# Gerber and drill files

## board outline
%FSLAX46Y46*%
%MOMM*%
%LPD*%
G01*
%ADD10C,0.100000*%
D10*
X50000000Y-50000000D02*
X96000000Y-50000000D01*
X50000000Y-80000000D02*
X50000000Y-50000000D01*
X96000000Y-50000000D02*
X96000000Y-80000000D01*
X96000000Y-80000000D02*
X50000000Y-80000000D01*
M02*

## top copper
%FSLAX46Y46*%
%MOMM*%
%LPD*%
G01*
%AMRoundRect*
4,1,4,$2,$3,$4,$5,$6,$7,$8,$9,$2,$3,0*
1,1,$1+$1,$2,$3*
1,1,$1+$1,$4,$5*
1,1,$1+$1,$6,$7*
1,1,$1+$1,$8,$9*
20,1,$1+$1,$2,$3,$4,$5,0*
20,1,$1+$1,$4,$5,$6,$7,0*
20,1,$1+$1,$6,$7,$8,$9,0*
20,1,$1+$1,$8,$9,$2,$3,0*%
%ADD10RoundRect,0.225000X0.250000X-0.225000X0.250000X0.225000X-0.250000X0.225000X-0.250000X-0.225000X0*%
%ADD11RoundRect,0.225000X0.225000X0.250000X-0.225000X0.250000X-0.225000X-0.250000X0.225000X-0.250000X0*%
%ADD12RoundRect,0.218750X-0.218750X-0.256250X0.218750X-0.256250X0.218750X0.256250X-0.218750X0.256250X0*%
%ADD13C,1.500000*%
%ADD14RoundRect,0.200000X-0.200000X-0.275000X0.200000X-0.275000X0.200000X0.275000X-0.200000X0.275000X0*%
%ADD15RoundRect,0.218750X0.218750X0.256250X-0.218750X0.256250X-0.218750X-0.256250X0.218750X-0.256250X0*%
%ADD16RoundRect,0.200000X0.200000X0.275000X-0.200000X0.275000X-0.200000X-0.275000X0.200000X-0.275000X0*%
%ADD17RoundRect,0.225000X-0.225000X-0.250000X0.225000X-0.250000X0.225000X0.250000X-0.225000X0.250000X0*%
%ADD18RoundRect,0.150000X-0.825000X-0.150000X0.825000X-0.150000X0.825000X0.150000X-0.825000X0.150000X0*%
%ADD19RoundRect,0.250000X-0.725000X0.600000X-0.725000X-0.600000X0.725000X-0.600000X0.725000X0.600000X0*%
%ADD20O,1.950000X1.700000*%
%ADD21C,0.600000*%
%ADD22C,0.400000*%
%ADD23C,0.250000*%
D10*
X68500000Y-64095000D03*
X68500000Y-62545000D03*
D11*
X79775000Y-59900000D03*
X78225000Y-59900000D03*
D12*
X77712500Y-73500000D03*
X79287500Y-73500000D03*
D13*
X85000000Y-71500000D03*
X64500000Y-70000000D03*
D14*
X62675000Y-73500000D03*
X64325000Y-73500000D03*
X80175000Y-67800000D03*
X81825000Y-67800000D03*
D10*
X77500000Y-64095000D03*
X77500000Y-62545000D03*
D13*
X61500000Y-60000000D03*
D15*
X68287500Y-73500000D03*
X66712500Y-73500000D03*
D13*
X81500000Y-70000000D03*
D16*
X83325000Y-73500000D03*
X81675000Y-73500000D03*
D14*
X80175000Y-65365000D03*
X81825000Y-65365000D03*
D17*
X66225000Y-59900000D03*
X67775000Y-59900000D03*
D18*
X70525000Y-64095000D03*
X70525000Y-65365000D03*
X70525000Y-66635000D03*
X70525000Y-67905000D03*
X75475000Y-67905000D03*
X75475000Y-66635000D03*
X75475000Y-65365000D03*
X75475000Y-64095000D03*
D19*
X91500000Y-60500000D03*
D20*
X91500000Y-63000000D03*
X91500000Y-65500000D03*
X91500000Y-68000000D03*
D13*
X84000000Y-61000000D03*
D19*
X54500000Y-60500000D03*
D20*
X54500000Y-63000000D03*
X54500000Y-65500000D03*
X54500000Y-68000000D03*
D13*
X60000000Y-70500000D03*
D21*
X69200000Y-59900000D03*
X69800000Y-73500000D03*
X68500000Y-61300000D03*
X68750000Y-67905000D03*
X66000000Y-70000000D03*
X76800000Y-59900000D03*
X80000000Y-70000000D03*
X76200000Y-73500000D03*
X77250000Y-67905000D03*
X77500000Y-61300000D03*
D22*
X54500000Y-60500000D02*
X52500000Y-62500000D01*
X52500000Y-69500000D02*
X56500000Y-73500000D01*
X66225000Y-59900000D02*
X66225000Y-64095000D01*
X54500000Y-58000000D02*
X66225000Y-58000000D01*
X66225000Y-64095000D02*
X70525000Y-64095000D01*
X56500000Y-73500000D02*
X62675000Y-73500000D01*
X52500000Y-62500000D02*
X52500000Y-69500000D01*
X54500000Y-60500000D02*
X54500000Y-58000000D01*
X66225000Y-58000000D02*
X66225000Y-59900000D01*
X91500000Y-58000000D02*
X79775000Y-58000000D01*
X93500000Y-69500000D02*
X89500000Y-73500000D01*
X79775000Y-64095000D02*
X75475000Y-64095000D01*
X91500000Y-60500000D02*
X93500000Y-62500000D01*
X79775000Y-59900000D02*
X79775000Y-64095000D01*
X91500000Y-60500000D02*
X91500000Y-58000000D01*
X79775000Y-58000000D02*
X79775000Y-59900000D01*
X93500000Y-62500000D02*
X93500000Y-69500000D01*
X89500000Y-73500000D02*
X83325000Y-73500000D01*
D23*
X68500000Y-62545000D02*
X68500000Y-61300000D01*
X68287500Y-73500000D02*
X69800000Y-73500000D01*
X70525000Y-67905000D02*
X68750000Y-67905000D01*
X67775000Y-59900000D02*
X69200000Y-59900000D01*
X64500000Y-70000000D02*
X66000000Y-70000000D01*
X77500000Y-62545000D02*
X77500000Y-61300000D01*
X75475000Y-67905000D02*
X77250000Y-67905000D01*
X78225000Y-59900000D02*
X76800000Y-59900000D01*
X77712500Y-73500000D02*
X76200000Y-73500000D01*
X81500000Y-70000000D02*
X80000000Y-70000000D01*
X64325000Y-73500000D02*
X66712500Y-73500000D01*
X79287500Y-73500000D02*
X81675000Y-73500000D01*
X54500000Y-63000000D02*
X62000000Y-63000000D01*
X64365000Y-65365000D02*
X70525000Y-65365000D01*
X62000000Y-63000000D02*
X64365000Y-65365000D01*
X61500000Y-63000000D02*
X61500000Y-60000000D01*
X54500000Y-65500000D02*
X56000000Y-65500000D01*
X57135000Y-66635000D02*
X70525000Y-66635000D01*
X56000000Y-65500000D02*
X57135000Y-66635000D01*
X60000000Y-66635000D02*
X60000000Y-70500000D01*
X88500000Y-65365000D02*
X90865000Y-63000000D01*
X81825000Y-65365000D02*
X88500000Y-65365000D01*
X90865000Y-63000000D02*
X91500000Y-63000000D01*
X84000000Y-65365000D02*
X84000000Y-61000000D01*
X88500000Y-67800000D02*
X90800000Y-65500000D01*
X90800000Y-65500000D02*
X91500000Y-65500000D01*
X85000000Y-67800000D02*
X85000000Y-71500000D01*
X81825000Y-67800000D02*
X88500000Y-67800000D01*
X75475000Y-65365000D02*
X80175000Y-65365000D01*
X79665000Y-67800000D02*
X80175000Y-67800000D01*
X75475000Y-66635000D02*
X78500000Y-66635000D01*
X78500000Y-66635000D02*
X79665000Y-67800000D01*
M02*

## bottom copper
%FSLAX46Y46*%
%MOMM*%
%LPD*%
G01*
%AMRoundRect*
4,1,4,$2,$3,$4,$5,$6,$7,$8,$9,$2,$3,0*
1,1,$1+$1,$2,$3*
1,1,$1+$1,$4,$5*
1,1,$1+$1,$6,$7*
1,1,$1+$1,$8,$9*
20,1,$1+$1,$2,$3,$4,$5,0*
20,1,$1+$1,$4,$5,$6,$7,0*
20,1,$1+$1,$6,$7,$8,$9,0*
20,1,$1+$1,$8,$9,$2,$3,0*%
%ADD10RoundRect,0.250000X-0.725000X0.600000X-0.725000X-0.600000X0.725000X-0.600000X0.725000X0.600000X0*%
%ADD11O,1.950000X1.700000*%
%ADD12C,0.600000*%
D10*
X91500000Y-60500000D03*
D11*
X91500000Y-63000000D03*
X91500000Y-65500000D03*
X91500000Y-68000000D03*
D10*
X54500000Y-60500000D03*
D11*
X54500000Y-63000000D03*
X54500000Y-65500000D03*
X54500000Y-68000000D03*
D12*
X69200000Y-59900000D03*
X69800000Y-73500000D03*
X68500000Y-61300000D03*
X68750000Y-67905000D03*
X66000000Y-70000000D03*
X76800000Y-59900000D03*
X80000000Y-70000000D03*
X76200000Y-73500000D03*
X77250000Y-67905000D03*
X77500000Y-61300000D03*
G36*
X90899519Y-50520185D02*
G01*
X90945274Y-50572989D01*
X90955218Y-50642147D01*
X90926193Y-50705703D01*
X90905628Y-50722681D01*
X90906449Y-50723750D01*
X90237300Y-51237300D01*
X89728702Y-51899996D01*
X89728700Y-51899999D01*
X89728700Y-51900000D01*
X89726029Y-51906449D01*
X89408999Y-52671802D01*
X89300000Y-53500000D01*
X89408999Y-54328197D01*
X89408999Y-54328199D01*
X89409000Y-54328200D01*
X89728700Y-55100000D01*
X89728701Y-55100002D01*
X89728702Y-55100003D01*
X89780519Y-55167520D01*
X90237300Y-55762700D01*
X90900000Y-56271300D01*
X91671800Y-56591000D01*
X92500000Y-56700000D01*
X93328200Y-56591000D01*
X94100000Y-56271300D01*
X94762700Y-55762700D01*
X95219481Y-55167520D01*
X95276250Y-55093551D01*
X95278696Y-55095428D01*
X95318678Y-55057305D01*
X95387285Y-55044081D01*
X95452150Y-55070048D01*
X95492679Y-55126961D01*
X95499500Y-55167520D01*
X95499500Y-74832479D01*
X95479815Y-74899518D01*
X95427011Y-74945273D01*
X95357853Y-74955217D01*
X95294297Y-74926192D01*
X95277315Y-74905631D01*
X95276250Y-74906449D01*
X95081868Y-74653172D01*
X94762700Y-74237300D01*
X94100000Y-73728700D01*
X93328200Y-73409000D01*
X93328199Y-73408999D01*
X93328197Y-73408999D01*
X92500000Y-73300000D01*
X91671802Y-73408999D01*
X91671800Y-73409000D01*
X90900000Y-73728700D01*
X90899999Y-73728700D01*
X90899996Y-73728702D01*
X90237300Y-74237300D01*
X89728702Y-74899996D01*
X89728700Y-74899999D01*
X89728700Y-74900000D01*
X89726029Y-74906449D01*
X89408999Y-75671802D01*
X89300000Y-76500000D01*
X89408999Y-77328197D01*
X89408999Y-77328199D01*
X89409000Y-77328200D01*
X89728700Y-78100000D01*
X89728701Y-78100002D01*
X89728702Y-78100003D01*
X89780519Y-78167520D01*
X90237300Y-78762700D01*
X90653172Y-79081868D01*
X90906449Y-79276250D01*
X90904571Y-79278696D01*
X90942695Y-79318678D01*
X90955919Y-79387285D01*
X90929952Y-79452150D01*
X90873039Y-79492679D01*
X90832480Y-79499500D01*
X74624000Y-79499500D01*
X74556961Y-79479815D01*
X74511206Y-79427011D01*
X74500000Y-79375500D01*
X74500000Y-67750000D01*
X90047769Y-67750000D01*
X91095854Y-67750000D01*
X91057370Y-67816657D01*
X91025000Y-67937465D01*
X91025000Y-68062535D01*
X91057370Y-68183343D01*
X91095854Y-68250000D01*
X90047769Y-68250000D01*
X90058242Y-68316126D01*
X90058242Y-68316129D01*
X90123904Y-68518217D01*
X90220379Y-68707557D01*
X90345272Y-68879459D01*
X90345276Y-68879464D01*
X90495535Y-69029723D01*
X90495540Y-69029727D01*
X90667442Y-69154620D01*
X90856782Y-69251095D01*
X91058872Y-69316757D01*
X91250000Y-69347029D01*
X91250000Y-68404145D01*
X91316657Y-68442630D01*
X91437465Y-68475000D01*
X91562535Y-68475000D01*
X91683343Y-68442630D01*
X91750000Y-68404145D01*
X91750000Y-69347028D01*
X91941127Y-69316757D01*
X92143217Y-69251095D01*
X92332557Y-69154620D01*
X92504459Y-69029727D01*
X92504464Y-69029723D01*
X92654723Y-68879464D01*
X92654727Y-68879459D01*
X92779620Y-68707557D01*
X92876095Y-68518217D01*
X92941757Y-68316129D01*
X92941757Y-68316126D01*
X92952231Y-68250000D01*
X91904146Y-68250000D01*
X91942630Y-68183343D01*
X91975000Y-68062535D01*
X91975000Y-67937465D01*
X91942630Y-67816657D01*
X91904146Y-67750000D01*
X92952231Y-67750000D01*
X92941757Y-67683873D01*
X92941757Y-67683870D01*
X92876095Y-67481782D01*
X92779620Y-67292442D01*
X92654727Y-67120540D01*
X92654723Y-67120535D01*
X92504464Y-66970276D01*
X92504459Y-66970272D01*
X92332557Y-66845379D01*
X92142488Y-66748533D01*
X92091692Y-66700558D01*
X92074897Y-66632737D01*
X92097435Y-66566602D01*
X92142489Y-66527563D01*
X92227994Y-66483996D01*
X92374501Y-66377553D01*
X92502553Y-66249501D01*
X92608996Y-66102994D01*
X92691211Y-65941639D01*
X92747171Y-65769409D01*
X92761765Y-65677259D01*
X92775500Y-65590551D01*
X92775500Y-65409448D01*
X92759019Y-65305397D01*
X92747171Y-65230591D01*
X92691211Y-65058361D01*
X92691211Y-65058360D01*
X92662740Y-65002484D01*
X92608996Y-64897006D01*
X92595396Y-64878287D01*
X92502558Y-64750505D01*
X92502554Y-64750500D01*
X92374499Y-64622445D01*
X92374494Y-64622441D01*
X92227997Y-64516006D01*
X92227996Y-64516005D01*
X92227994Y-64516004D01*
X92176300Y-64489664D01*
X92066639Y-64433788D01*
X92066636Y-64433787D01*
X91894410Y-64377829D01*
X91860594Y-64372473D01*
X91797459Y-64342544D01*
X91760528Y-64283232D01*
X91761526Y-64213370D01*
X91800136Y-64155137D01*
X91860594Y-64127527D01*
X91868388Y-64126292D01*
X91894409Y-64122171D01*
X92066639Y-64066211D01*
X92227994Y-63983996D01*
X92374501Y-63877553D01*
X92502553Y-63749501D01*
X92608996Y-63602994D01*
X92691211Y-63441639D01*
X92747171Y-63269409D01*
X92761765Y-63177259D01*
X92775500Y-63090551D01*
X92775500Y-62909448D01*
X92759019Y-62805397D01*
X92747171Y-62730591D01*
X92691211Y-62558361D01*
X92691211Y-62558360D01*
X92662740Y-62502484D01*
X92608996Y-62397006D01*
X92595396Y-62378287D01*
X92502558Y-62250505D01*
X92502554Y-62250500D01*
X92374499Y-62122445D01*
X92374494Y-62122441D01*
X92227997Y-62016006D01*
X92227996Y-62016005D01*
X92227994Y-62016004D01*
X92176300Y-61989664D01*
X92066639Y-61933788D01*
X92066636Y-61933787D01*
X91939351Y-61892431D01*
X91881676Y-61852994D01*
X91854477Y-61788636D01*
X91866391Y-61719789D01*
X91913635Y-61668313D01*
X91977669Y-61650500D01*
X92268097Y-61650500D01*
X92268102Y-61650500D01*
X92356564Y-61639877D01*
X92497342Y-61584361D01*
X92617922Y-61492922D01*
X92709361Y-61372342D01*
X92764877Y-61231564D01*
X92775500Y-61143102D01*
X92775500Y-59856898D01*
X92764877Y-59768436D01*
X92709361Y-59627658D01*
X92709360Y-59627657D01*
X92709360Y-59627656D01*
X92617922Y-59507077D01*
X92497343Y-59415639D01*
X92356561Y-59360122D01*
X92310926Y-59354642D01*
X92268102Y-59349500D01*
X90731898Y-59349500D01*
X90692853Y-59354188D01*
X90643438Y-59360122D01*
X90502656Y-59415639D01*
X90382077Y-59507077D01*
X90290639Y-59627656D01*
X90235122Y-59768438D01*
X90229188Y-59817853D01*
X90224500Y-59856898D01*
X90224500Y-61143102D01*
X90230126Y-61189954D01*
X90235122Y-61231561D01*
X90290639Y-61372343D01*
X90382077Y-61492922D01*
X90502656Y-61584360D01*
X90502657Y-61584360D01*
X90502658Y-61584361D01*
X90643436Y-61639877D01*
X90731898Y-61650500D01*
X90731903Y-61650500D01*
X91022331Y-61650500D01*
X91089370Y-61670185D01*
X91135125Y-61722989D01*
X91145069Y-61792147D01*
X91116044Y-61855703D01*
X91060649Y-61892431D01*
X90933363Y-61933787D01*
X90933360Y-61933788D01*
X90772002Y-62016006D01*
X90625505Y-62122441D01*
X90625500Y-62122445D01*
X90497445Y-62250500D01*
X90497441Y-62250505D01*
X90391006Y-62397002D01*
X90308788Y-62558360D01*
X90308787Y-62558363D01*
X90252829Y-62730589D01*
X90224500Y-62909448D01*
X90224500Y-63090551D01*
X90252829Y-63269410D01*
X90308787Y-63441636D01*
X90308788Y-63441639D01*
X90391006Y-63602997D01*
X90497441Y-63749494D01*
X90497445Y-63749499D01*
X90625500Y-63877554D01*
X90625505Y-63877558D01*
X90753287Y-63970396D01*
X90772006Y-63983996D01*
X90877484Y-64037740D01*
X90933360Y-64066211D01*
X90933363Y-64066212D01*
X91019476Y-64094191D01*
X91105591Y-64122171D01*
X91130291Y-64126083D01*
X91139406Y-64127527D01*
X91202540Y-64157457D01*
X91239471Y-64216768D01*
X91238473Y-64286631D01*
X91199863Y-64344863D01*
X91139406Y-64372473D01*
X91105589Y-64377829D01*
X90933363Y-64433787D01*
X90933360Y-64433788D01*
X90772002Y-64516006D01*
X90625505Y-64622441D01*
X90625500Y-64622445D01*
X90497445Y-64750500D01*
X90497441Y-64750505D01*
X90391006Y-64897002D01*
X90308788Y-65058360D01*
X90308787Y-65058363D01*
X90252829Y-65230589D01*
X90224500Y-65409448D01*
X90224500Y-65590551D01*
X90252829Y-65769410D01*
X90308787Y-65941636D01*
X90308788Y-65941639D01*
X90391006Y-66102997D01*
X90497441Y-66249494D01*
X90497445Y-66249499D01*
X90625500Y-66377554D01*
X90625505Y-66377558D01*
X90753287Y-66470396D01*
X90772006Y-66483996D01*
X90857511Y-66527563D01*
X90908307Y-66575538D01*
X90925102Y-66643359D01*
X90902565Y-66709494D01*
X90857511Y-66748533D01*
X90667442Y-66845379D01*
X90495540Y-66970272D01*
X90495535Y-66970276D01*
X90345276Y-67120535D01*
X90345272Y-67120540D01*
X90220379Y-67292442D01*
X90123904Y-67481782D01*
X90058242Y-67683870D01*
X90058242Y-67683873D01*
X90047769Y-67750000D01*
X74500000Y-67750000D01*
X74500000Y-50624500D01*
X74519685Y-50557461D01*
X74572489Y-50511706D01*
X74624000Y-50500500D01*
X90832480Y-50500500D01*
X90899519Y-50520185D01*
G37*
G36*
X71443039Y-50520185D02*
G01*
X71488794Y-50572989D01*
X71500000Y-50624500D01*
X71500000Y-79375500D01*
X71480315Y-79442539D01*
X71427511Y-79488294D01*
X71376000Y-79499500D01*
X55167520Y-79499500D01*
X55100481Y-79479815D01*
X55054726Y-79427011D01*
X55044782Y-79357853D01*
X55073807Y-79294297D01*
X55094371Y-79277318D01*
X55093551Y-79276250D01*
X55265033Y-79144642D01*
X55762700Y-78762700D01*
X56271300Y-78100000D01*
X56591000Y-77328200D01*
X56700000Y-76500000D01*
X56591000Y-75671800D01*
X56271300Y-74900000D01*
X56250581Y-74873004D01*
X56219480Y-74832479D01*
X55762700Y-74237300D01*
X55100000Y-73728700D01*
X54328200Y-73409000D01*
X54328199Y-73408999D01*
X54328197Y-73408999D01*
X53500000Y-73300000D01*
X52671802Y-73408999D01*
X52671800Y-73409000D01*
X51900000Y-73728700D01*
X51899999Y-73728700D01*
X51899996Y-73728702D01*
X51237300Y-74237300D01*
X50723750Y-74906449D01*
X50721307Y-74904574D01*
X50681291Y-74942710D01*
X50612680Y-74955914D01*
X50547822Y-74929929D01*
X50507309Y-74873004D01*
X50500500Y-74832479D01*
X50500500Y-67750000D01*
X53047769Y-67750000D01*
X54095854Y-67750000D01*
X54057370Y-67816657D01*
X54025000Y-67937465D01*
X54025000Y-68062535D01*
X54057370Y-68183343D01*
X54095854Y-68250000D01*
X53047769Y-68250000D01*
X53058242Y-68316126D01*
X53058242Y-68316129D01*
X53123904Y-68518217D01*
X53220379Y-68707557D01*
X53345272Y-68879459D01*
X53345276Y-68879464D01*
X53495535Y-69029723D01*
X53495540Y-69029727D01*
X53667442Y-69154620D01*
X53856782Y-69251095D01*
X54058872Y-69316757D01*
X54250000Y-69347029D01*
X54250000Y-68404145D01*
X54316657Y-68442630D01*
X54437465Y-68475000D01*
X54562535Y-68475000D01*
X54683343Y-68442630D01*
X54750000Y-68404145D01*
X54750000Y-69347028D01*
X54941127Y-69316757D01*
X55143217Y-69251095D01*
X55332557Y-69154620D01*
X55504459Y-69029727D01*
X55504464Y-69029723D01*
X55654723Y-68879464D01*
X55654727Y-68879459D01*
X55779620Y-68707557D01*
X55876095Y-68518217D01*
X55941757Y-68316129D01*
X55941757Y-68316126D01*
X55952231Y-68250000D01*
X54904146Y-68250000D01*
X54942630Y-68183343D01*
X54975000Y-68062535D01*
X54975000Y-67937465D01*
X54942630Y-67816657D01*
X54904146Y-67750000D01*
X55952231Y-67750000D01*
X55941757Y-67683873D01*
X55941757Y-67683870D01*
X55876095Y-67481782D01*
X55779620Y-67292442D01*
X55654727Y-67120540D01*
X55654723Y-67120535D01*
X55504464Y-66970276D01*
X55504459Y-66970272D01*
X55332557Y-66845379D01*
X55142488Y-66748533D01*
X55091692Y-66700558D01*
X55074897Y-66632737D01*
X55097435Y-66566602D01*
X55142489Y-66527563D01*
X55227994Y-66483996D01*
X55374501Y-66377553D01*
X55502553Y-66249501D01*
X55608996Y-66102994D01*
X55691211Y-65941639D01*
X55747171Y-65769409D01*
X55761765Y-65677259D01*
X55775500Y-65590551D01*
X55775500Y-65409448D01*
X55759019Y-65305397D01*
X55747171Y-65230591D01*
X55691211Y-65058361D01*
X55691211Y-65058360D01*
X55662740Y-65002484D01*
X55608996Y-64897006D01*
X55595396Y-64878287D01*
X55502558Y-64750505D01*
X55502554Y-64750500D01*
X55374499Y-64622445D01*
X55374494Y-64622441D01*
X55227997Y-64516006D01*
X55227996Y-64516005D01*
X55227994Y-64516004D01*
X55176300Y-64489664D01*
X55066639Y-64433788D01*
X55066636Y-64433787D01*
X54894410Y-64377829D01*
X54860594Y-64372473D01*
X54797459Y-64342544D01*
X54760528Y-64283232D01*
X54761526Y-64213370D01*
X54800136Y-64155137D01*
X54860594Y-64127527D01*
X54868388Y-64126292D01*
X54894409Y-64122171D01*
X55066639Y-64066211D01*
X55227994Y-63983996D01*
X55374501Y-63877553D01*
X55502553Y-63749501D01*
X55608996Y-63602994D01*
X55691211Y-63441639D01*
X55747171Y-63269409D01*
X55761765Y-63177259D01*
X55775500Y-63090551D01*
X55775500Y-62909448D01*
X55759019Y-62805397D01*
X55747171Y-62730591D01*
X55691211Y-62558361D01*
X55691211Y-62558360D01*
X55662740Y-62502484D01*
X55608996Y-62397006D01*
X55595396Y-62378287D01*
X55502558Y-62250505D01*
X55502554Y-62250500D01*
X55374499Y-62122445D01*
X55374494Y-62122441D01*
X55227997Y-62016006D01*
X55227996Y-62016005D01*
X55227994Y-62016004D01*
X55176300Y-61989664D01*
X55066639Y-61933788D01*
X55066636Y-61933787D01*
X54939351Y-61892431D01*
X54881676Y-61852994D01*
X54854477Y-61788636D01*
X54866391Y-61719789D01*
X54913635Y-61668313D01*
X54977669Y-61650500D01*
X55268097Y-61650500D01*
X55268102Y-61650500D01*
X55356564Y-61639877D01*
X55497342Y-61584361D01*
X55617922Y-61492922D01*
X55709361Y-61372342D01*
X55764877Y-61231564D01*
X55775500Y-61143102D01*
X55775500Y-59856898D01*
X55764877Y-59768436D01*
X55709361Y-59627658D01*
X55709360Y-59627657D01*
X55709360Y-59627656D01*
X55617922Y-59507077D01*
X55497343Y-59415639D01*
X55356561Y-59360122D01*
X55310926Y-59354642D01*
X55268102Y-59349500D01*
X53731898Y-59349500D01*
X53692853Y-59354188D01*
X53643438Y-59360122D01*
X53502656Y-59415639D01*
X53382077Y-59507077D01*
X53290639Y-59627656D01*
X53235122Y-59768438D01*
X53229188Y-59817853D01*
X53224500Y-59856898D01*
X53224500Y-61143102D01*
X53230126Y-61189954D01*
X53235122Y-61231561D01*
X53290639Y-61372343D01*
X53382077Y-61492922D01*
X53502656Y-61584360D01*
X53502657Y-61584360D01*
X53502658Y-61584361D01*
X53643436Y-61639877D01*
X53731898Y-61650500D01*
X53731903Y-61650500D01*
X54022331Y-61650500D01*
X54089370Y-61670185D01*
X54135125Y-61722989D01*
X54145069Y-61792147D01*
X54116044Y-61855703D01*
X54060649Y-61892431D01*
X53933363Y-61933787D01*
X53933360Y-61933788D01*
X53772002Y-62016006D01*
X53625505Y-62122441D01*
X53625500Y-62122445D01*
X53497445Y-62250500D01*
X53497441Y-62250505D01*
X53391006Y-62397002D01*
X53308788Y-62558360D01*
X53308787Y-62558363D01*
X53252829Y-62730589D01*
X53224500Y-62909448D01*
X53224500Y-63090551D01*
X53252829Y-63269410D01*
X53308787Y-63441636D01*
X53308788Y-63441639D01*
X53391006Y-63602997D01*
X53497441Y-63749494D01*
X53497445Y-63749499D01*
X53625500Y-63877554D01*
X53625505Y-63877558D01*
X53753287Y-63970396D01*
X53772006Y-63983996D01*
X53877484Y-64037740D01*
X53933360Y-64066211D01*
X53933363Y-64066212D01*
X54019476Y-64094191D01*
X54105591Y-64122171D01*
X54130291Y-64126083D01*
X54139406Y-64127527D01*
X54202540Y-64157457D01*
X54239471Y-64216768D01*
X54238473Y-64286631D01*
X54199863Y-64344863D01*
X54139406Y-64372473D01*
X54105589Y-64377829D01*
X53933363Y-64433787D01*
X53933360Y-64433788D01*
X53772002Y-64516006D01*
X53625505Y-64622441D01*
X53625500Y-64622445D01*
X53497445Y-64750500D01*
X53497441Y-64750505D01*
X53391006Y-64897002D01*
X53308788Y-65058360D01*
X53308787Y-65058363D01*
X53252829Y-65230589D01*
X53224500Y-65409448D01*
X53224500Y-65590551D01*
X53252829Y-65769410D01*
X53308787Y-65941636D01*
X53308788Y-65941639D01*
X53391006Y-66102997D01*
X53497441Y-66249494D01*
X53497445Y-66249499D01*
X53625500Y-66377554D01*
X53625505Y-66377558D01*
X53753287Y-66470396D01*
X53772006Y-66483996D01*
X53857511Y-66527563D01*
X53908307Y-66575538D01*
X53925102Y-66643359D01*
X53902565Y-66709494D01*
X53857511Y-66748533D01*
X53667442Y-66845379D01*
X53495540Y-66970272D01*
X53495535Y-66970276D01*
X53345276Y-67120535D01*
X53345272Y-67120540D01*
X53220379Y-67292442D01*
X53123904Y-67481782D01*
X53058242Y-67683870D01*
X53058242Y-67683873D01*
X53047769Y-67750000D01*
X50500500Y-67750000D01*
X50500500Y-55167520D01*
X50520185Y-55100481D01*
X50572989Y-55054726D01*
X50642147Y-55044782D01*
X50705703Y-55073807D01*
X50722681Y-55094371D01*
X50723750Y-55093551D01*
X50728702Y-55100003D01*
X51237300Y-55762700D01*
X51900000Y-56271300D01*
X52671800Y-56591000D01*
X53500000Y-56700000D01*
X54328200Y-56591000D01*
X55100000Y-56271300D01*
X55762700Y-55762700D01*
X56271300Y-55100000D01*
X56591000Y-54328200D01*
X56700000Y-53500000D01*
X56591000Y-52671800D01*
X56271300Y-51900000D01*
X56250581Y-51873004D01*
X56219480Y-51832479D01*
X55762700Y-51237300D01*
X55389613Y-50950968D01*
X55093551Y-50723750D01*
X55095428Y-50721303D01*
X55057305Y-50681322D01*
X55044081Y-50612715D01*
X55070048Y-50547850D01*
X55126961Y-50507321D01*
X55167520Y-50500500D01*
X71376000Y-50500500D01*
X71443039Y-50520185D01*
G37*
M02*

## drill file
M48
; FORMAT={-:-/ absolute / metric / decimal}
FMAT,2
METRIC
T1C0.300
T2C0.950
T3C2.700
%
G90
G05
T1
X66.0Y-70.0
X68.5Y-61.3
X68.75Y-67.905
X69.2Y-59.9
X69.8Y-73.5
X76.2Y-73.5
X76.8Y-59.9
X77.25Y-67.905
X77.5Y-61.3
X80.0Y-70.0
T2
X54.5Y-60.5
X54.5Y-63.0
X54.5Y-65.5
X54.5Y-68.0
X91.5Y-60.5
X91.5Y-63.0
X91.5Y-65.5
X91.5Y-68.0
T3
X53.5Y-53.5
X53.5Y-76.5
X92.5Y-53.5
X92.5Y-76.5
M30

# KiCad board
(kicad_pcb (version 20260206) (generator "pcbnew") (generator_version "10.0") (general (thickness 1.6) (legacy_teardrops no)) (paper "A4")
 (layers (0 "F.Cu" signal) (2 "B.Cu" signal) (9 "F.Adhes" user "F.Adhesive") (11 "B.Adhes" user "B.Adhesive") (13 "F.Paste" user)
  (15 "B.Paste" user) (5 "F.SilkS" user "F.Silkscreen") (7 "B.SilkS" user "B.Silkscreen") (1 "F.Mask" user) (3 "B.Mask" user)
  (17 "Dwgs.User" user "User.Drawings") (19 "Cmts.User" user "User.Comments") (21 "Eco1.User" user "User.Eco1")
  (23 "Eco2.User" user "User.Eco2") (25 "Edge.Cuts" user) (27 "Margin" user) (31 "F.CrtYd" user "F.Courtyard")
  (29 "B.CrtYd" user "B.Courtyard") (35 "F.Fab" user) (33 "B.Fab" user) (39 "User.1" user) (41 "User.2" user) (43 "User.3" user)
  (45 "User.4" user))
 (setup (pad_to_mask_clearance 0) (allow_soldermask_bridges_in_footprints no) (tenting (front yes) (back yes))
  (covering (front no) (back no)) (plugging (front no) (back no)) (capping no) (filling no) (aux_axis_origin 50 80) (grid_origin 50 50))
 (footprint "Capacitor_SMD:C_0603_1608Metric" (layer "F.Cu") (at 68.5 63.32 90)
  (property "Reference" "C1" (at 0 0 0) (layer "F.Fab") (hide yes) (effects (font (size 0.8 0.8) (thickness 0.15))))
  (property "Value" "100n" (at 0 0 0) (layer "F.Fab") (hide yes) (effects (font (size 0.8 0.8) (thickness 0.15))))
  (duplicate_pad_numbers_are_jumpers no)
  (pad "1" smd roundrect (at -0.775 0 90) (size 0.9 0.95) (layers "F.Cu" "F.Mask" "F.Paste") (roundrect_rratio 0.25) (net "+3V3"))
  (pad "2" smd roundrect (at 0.775 0 90) (size 0.9 0.95) (layers "F.Cu" "F.Mask" "F.Paste") (roundrect_rratio 0.25) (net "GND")))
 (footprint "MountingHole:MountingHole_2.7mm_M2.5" (layer "F.Cu") (at 92.5 53.5)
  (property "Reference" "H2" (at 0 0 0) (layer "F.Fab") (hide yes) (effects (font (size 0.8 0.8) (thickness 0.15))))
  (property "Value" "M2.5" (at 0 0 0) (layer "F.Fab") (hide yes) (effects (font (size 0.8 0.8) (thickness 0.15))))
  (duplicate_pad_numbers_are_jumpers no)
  (pad "" np_thru_hole circle (at 0 0) (size 2.7 2.7) (drill 2.7) (layers "*.Cu" "*.Mask")))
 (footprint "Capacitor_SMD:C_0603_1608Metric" (layer "F.Cu") (at 79 59.9 180)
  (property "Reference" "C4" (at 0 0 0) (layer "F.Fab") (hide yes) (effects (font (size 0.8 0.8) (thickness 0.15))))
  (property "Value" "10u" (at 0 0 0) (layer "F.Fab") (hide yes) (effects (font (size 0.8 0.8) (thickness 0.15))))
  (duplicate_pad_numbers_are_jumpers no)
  (pad "1" smd roundrect (at -0.775 0 180) (size 0.9 0.95) (layers "F.Cu" "F.Mask" "F.Paste") (roundrect_rratio 0.25) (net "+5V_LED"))
  (pad "2" smd roundrect (at 0.775 0 180) (size 0.9 0.95) (layers "F.Cu" "F.Mask" "F.Paste") (roundrect_rratio 0.25) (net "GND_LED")))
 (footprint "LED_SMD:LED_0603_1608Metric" (layer "F.Cu") (at 78.5 73.5)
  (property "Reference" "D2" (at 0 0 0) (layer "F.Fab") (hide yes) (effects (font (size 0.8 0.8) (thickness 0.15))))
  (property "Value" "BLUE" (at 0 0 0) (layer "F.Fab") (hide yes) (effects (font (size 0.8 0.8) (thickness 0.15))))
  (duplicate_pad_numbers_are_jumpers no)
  (pad "1" smd roundrect (at -0.7875 0) (size 0.875 0.95) (layers "F.Cu" "F.Mask" "F.Paste") (roundrect_rratio 0.25) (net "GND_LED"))
  (pad "2" smd roundrect (at 0.7875 0) (size 0.875 0.95) (layers "F.Cu" "F.Mask" "F.Paste") (roundrect_rratio 0.25) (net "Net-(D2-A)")))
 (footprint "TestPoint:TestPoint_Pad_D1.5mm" (layer "F.Cu") (at 85 71.5)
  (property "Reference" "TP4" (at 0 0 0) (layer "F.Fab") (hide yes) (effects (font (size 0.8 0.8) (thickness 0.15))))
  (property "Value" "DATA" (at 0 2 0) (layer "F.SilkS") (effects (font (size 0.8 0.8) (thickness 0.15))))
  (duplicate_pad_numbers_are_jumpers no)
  (pad "1" smd circle (at 0 0) (size 1.5 1.5) (layers "F.Cu" "F.Mask") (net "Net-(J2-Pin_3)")))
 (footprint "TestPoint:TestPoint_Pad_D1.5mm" (layer "F.Cu") (at 64.5 70)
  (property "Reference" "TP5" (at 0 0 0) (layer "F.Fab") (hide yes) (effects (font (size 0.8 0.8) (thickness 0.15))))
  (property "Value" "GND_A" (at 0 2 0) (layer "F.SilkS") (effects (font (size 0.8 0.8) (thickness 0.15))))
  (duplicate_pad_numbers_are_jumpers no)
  (pad "1" smd circle (at 0 0) (size 1.5 1.5) (layers "F.Cu" "F.Mask") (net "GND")))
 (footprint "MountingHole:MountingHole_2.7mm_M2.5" (layer "F.Cu") (at 92.5 76.5)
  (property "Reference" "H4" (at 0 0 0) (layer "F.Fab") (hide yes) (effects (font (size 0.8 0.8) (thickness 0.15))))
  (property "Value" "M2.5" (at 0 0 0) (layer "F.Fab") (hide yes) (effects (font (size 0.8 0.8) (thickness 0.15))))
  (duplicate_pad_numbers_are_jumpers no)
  (pad "" np_thru_hole circle (at 0 0) (size 2.7 2.7) (drill 2.7) (layers "*.Cu" "*.Mask")))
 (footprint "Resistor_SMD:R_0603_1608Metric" (layer "F.Cu") (at 63.5 73.5)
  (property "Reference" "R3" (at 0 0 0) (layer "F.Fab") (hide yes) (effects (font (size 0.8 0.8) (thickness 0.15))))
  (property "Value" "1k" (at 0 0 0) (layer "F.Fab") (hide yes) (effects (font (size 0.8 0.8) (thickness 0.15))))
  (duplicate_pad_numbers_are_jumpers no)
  (pad "1" smd roundrect (at -0.825 0) (size 0.8 0.95) (layers "F.Cu" "F.Mask" "F.Paste") (roundrect_rratio 0.25) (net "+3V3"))
  (pad "2" smd roundrect (at 0.825 0) (size 0.8 0.95) (layers "F.Cu" "F.Mask" "F.Paste") (roundrect_rratio 0.25) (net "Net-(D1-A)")))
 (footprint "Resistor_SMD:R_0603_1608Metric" (layer "F.Cu") (at 81 67.8)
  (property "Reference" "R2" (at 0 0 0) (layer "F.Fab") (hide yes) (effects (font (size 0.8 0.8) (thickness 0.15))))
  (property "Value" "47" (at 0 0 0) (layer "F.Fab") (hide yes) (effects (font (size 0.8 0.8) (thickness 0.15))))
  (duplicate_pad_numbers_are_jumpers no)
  (pad "1" smd roundrect (at -0.825 0) (size 0.8 0.95) (layers "F.Cu" "F.Mask" "F.Paste") (roundrect_rratio 0.25) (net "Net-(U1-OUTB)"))
  (pad "2" smd roundrect (at 0.825 0) (size 0.8 0.95) (layers "F.Cu" "F.Mask" "F.Paste") (roundrect_rratio 0.25) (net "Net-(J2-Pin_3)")))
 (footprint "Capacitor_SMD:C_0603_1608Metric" (layer "F.Cu") (at 77.5 63.32 90)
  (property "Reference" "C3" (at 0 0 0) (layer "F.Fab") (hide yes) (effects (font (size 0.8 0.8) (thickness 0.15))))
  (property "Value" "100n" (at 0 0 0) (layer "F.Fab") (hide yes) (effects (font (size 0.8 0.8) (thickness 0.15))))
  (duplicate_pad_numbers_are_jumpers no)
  (pad "1" smd roundrect (at -0.775 0 90) (size 0.9 0.95) (layers "F.Cu" "F.Mask" "F.Paste") (roundrect_rratio 0.25) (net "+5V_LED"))
  (pad "2" smd roundrect (at 0.775 0 90) (size 0.9 0.95) (layers "F.Cu" "F.Mask" "F.Paste") (roundrect_rratio 0.25) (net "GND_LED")))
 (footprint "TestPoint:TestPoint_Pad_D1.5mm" (layer "F.Cu") (at 61.5 60)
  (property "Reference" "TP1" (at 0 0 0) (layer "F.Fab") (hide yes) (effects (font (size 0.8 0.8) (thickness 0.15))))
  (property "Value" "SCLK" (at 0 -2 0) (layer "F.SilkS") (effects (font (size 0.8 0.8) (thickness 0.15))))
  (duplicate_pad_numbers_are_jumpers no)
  (pad "1" smd circle (at 0 0) (size 1.5 1.5) (layers "F.Cu" "F.Mask") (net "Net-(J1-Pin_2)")))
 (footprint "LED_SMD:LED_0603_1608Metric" (layer "F.Cu") (at 67.5 73.5 180)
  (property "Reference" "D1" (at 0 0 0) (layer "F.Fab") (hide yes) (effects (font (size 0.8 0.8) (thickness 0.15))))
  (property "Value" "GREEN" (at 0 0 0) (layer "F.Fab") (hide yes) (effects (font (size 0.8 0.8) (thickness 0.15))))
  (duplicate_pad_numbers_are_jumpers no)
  (pad "1" smd roundrect (at -0.7875 0 180) (size 0.875 0.95) (layers "F.Cu" "F.Mask" "F.Paste") (roundrect_rratio 0.25) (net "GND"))
  (pad "2" smd roundrect (at 0.7875 0 180) (size 0.875 0.95) (layers "F.Cu" "F.Mask" "F.Paste") (roundrect_rratio 0.25) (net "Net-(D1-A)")))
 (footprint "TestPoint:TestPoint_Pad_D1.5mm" (layer "F.Cu") (at 81.5 70)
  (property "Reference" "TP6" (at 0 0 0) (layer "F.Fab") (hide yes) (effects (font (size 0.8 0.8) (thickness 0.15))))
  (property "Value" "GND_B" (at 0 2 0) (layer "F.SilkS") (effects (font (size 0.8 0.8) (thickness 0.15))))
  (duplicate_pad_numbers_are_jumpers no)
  (pad "1" smd circle (at 0 0) (size 1.5 1.5) (layers "F.Cu" "F.Mask") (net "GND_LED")))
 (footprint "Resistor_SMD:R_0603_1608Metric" (layer "F.Cu") (at 82.5 73.5 180)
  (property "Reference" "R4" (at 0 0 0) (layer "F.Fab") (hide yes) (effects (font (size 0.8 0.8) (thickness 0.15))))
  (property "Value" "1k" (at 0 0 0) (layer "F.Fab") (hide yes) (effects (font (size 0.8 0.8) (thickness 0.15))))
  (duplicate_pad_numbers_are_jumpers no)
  (pad "1" smd roundrect (at -0.825 0 180) (size 0.8 0.95) (layers "F.Cu" "F.Mask" "F.Paste") (roundrect_rratio 0.25) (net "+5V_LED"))
  (pad "2" smd roundrect (at 0.825 0 180) (size 0.8 0.95) (layers "F.Cu" "F.Mask" "F.Paste") (roundrect_rratio 0.25) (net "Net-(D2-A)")))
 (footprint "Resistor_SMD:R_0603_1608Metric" (layer "F.Cu") (at 81 65.365)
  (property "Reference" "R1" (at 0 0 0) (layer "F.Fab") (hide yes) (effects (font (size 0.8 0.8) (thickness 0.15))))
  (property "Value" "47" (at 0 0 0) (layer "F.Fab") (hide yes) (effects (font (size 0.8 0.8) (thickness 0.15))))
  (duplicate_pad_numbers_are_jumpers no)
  (pad "1" smd roundrect (at -0.825 0) (size 0.8 0.95) (layers "F.Cu" "F.Mask" "F.Paste") (roundrect_rratio 0.25) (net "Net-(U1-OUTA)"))
  (pad "2" smd roundrect (at 0.825 0) (size 0.8 0.95) (layers "F.Cu" "F.Mask" "F.Paste") (roundrect_rratio 0.25) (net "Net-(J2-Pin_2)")))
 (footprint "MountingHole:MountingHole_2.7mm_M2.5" (layer "F.Cu") (at 53.5 76.5)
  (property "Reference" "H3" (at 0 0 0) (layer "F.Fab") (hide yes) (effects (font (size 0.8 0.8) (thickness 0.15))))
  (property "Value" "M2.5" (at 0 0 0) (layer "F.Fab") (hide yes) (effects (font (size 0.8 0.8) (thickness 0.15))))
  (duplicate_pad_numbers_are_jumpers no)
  (pad "" np_thru_hole circle (at 0 0) (size 2.7 2.7) (drill 2.7) (layers "*.Cu" "*.Mask")))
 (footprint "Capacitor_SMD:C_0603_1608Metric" (layer "F.Cu") (at 67 59.9)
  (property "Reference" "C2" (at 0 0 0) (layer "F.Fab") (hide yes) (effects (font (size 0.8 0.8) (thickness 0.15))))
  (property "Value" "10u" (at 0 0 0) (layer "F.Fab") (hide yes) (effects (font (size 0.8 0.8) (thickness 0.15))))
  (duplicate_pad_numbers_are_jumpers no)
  (pad "1" smd roundrect (at -0.775 0) (size 0.9 0.95) (layers "F.Cu" "F.Mask" "F.Paste") (roundrect_rratio 0.25) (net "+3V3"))
  (pad "2" smd roundrect (at 0.775 0) (size 0.9 0.95) (layers "F.Cu" "F.Mask" "F.Paste") (roundrect_rratio 0.25) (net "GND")))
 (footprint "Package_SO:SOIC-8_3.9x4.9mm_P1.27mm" (layer "F.Cu") (at 73 66)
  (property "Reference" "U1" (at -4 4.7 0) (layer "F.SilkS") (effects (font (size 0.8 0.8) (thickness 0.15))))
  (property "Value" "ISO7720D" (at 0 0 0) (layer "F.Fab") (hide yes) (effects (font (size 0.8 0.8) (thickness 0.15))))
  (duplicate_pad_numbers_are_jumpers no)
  (pad "1" smd roundrect (at -2.475 -1.905) (size 1.95 0.6) (layers "F.Cu" "F.Mask" "F.Paste") (roundrect_rratio 0.25) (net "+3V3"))
  (pad "2" smd roundrect (at -2.475 -0.635) (size 1.95 0.6) (layers "F.Cu" "F.Mask" "F.Paste") (roundrect_rratio 0.25)
   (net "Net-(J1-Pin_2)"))
  (pad "3" smd roundrect (at -2.475 0.635) (size 1.95 0.6) (layers "F.Cu" "F.Mask" "F.Paste") (roundrect_rratio 0.25) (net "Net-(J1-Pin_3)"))
  (pad "4" smd roundrect (at -2.475 1.905) (size 1.95 0.6) (layers "F.Cu" "F.Mask" "F.Paste") (roundrect_rratio 0.25) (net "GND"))
  (pad "5" smd roundrect (at 2.475 1.905) (size 1.95 0.6) (layers "F.Cu" "F.Mask" "F.Paste") (roundrect_rratio 0.25) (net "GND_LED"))
  (pad "6" smd roundrect (at 2.475 0.635) (size 1.95 0.6) (layers "F.Cu" "F.Mask" "F.Paste") (roundrect_rratio 0.25) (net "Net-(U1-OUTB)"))
  (pad "7" smd roundrect (at 2.475 -0.635) (size 1.95 0.6) (layers "F.Cu" "F.Mask" "F.Paste") (roundrect_rratio 0.25) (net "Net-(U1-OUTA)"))
  (pad "8" smd roundrect (at 2.475 -1.905) (size 1.95 0.6) (layers "F.Cu" "F.Mask" "F.Paste") (roundrect_rratio 0.25) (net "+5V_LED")))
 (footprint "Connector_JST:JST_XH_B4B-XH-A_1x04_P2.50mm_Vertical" (layer "F.Cu") (at 91.5 60.5 -90)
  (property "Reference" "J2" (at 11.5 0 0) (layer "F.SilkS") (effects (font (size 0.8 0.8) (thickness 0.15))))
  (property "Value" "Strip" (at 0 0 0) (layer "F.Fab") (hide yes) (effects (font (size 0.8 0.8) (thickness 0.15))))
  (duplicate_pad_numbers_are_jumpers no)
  (pad "1" thru_hole roundrect (at 0 0 270) (size 1.7 1.95) (drill 0.95) (layers "*.Cu" "*.Mask") (remove_unused_layers no)
   (roundrect_rratio 0.147059) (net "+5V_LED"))
  (pad "2" thru_hole oval (at 2.5 0 270) (size 1.7 1.95) (drill 0.95) (layers "*.Cu" "*.Mask") (remove_unused_layers no)
   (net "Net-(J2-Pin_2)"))
  (pad "3" thru_hole oval (at 5 0 270) (size 1.7 1.95) (drill 0.95) (layers "*.Cu" "*.Mask") (remove_unused_layers no)
   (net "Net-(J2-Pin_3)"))
  (pad "4" thru_hole oval (at 7.5 0 270) (size 1.7 1.95) (drill 0.95) (layers "*.Cu" "*.Mask") (remove_unused_layers no) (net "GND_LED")))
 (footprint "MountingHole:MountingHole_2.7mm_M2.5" (layer "F.Cu") (at 53.5 53.5)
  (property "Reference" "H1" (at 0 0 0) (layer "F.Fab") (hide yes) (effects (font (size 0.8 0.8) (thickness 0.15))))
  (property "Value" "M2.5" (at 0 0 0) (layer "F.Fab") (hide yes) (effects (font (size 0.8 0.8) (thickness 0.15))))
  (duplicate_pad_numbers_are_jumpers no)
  (pad "" np_thru_hole circle (at 0 0) (size 2.7 2.7) (drill 2.7) (layers "*.Cu" "*.Mask")))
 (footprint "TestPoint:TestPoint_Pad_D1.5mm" (layer "F.Cu") (at 84 61)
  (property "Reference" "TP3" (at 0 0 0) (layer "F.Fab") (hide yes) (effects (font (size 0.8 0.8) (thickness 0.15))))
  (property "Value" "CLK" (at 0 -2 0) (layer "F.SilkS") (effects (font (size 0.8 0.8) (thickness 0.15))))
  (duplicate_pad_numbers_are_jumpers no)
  (pad "1" smd circle (at 0 0) (size 1.5 1.5) (layers "F.Cu" "F.Mask") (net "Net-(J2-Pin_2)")))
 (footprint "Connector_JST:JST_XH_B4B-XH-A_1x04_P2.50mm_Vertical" (layer "F.Cu") (at 54.5 60.5 -90)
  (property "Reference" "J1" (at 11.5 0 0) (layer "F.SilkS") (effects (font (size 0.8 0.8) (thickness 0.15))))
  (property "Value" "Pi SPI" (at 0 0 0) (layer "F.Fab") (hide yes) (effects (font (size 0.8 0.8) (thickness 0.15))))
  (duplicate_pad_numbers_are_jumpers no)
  (pad "1" thru_hole roundrect (at 0 0 270) (size 1.7 1.95) (drill 0.95) (layers "*.Cu" "*.Mask") (remove_unused_layers no)
   (roundrect_rratio 0.147059) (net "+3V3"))
  (pad "2" thru_hole oval (at 2.5 0 270) (size 1.7 1.95) (drill 0.95) (layers "*.Cu" "*.Mask") (remove_unused_layers no)
   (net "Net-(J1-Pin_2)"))
  (pad "3" thru_hole oval (at 5 0 270) (size 1.7 1.95) (drill 0.95) (layers "*.Cu" "*.Mask") (remove_unused_layers no)
   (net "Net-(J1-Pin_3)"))
  (pad "4" thru_hole oval (at 7.5 0 270) (size 1.7 1.95) (drill 0.95) (layers "*.Cu" "*.Mask") (remove_unused_layers no) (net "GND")))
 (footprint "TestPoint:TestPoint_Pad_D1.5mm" (layer "F.Cu") (at 60 70.5)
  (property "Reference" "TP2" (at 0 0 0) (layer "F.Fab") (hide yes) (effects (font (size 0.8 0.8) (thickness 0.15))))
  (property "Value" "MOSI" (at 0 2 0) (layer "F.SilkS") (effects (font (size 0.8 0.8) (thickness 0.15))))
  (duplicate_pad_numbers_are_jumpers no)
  (pad "1" smd circle (at 0 0) (size 1.5 1.5) (layers "F.Cu" "F.Mask") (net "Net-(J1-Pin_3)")))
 (gr_line (start 50 50) (end 96 50) (stroke (width 0.1) (type default)) (layer "Edge.Cuts"))
 (gr_line (start 50 80) (end 50 50) (stroke (width 0.1) (type default)) (layer "Edge.Cuts"))
 (gr_line (start 96 50) (end 96 80) (stroke (width 0.1) (type default)) (layer "Edge.Cuts"))
 (gr_line (start 96 80) (end 50 80) (stroke (width 0.1) (type default)) (layer "Edge.Cuts"))
 (segment (start 54.5 60.5) (end 52.5 62.5) (width 0.4) (layer "F.Cu") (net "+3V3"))
 (segment (start 52.5 69.5) (end 56.5 73.5) (width 0.4) (layer "F.Cu") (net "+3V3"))
 (segment (start 66.225 59.9) (end 66.225 64.095) (width 0.4) (layer "F.Cu") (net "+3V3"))
 (segment (start 54.5 58) (end 66.225 58) (width 0.4) (layer "F.Cu") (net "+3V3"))
 (segment (start 66.225 64.095) (end 70.525 64.095) (width 0.4) (layer "F.Cu") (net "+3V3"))
 (segment (start 56.5 73.5) (end 62.675 73.5) (width 0.4) (layer "F.Cu") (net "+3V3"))
 (segment (start 52.5 62.5) (end 52.5 69.5) (width 0.4) (layer "F.Cu") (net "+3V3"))
 (segment (start 54.5 60.5) (end 54.5 58) (width 0.4) (layer "F.Cu") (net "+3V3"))
 (segment (start 66.225 58) (end 66.225 59.9) (width 0.4) (layer "F.Cu") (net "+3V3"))
 (segment (start 91.5 58) (end 79.775 58) (width 0.4) (layer "F.Cu") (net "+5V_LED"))
 (segment (start 93.5 69.5) (end 89.5 73.5) (width 0.4) (layer "F.Cu") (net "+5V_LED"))
 (segment (start 79.775 64.095) (end 75.475 64.095) (width 0.4) (layer "F.Cu") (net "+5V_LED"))
 (segment (start 91.5 60.5) (end 93.5 62.5) (width 0.4) (layer "F.Cu") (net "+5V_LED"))
 (segment (start 79.775 59.9) (end 79.775 64.095) (width 0.4) (layer "F.Cu") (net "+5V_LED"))
 (segment (start 91.5 60.5) (end 91.5 58) (width 0.4) (layer "F.Cu") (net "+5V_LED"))
 (segment (start 79.775 58) (end 79.775 59.9) (width 0.4) (layer "F.Cu") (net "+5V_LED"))
 (segment (start 93.5 62.5) (end 93.5 69.5) (width 0.4) (layer "F.Cu") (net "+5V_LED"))
 (segment (start 89.5 73.5) (end 83.325 73.5) (width 0.4) (layer "F.Cu") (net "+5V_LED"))
 (segment (start 68.5 62.545) (end 68.5 61.3) (width 0.25) (layer "F.Cu") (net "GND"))
 (segment (start 68.2875 73.5) (end 69.8 73.5) (width 0.25) (layer "F.Cu") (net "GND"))
 (segment (start 70.525 67.905) (end 68.75 67.905) (width 0.25) (layer "F.Cu") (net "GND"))
 (segment (start 67.775 59.9) (end 69.2 59.9) (width 0.25) (layer "F.Cu") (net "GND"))
 (segment (start 64.5 70) (end 66 70) (width 0.25) (layer "F.Cu") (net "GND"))
 (via (at 69.2 59.9) (size 0.6) (drill 0.3) (layers "F.Cu" "B.Cu") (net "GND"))
 (via (at 69.8 73.5) (size 0.6) (drill 0.3) (layers "F.Cu" "B.Cu") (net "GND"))
 (via (at 68.5 61.3) (size 0.6) (drill 0.3) (layers "F.Cu" "B.Cu") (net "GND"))
 (via (at 68.75 67.905) (size 0.6) (drill 0.3) (layers "F.Cu" "B.Cu") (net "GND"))
 (via (at 66 70) (size 0.6) (drill 0.3) (layers "F.Cu" "B.Cu") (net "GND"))
 (segment (start 77.5 62.545) (end 77.5 61.3) (width 0.25) (layer "F.Cu") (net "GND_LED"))
 (segment (start 75.475 67.905) (end 77.25 67.905) (width 0.25) (layer "F.Cu") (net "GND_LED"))
 (segment (start 78.225 59.9) (end 76.8 59.9) (width 0.25) (layer "F.Cu") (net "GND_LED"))
 (segment (start 77.7125 73.5) (end 76.2 73.5) (width 0.25) (layer "F.Cu") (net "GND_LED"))
 (segment (start 81.5 70) (end 80 70) (width 0.25) (layer "F.Cu") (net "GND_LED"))
 (via (at 76.8 59.9) (size 0.6) (drill 0.3) (layers "F.Cu" "B.Cu") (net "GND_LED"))
 (via (at 80 70) (size 0.6) (drill 0.3) (layers "F.Cu" "B.Cu") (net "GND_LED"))
 (via (at 76.2 73.5) (size 0.6) (drill 0.3) (layers "F.Cu" "B.Cu") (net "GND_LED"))
 (via (at 77.25 67.905) (size 0.6) (drill 0.3) (layers "F.Cu" "B.Cu") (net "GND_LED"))
 (via (at 77.5 61.3) (size 0.6) (drill 0.3) (layers "F.Cu" "B.Cu") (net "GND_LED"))
 (segment (start 64.325 73.5) (end 66.7125 73.5) (width 0.25) (layer "F.Cu") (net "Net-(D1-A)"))
 (segment (start 79.2875 73.5) (end 81.675 73.5) (width 0.25) (layer "F.Cu") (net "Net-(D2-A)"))
 (segment (start 54.5 63) (end 62 63) (width 0.25) (layer "F.Cu") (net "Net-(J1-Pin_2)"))
 (segment (start 64.365 65.365) (end 70.525 65.365) (width 0.25) (layer "F.Cu") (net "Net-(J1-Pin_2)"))
 (segment (start 62 63) (end 64.365 65.365) (width 0.25) (layer "F.Cu") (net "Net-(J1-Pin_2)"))
 (segment (start 61.5 63) (end 61.5 60) (width 0.25) (layer "F.Cu") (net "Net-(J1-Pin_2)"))
 (segment (start 54.5 65.5) (end 56 65.5) (width 0.25) (layer "F.Cu") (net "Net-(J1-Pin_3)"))
 (segment (start 57.135 66.635) (end 70.525 66.635) (width 0.25) (layer "F.Cu") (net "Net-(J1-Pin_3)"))
 (segment (start 56 65.5) (end 57.135 66.635) (width 0.25) (layer "F.Cu") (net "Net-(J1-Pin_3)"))
 (segment (start 60 66.635) (end 60 70.5) (width 0.25) (layer "F.Cu") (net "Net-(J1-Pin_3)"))
 (segment (start 88.5 65.365) (end 90.865 63) (width 0.25) (layer "F.Cu") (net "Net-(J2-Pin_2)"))
 (segment (start 81.825 65.365) (end 88.5 65.365) (width 0.25) (layer "F.Cu") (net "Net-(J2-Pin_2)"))
 (segment (start 90.865 63) (end 91.5 63) (width 0.25) (layer "F.Cu") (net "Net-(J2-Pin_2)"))
 (segment (start 84 65.365) (end 84 61) (width 0.25) (layer "F.Cu") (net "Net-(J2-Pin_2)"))
 (segment (start 88.5 67.8) (end 90.8 65.5) (width 0.25) (layer "F.Cu") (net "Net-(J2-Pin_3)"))
 (segment (start 90.8 65.5) (end 91.5 65.5) (width 0.25) (layer "F.Cu") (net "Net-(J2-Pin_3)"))
 (segment (start 85 67.8) (end 85 71.5) (width 0.25) (layer "F.Cu") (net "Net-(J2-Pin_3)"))
 (segment (start 81.825 67.8) (end 88.5 67.8) (width 0.25) (layer "F.Cu") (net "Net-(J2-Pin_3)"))
 (segment (start 75.475 65.365) (end 80.175 65.365) (width 0.25) (layer "F.Cu") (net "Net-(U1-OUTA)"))
 (segment (start 79.665 67.8) (end 80.175 67.8) (width 0.25) (layer "F.Cu") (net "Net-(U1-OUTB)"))
 (segment (start 75.475 66.635) (end 78.5 66.635) (width 0.25) (layer "F.Cu") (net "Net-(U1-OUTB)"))
 (segment (start 78.5 66.635) (end 79.665 67.8) (width 0.25) (layer "F.Cu") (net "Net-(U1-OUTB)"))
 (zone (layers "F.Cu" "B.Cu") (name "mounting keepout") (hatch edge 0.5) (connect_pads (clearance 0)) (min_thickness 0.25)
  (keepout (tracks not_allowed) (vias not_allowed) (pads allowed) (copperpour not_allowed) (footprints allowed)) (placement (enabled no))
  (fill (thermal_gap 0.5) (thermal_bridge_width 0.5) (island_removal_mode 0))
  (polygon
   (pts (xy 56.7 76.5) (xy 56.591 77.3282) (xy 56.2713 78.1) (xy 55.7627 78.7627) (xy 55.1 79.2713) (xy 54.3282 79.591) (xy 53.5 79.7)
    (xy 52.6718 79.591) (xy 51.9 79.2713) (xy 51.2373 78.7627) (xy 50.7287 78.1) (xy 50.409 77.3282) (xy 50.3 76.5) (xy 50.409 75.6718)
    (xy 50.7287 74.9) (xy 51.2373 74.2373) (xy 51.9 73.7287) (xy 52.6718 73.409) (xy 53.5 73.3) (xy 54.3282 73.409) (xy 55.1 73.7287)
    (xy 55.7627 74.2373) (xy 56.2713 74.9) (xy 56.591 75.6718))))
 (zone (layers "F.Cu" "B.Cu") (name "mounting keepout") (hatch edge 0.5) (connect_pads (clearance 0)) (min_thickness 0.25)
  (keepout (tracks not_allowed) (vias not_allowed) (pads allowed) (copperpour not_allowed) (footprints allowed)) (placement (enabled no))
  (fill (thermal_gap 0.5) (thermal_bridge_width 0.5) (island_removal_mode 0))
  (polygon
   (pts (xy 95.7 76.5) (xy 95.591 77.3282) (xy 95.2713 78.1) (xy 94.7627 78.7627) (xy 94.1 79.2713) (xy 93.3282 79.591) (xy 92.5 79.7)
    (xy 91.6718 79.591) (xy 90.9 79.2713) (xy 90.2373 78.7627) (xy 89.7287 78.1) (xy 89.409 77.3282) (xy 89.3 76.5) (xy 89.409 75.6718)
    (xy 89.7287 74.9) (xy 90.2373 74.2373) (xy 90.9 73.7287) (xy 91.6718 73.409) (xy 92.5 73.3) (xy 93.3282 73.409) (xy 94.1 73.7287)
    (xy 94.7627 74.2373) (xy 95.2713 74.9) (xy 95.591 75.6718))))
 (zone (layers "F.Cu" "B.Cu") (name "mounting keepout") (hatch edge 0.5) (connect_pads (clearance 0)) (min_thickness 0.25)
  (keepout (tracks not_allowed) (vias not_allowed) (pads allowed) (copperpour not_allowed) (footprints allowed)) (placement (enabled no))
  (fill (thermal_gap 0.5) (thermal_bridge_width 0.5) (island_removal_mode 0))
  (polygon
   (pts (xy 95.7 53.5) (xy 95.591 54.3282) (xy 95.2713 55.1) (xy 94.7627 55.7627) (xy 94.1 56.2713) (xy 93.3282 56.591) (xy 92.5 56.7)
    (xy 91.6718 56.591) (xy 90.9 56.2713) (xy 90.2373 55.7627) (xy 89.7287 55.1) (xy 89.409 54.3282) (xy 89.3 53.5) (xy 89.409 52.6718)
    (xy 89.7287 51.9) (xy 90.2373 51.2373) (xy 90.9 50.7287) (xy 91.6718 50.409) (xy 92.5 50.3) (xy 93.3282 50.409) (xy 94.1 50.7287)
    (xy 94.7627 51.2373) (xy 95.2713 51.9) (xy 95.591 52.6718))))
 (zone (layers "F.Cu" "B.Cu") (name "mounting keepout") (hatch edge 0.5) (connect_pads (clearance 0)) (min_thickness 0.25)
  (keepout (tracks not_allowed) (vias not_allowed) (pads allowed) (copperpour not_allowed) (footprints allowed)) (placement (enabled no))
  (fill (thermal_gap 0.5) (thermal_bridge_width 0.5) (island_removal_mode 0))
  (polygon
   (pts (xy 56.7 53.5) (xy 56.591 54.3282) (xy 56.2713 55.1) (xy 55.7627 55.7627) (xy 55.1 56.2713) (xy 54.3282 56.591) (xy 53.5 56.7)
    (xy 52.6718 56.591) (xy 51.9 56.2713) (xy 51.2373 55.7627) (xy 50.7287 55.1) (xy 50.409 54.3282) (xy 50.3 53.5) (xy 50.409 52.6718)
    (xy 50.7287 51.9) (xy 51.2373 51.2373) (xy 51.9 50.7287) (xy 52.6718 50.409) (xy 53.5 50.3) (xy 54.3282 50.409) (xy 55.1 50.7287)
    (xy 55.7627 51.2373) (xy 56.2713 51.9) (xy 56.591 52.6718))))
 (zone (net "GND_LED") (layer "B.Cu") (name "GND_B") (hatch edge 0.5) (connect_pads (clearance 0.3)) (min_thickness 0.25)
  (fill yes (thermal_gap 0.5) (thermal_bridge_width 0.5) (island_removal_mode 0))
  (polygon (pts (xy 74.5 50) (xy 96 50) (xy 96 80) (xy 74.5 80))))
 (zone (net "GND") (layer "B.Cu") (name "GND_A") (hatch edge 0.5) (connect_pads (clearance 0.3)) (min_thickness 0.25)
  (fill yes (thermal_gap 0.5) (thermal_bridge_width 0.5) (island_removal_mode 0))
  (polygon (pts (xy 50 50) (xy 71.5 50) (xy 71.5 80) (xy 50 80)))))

